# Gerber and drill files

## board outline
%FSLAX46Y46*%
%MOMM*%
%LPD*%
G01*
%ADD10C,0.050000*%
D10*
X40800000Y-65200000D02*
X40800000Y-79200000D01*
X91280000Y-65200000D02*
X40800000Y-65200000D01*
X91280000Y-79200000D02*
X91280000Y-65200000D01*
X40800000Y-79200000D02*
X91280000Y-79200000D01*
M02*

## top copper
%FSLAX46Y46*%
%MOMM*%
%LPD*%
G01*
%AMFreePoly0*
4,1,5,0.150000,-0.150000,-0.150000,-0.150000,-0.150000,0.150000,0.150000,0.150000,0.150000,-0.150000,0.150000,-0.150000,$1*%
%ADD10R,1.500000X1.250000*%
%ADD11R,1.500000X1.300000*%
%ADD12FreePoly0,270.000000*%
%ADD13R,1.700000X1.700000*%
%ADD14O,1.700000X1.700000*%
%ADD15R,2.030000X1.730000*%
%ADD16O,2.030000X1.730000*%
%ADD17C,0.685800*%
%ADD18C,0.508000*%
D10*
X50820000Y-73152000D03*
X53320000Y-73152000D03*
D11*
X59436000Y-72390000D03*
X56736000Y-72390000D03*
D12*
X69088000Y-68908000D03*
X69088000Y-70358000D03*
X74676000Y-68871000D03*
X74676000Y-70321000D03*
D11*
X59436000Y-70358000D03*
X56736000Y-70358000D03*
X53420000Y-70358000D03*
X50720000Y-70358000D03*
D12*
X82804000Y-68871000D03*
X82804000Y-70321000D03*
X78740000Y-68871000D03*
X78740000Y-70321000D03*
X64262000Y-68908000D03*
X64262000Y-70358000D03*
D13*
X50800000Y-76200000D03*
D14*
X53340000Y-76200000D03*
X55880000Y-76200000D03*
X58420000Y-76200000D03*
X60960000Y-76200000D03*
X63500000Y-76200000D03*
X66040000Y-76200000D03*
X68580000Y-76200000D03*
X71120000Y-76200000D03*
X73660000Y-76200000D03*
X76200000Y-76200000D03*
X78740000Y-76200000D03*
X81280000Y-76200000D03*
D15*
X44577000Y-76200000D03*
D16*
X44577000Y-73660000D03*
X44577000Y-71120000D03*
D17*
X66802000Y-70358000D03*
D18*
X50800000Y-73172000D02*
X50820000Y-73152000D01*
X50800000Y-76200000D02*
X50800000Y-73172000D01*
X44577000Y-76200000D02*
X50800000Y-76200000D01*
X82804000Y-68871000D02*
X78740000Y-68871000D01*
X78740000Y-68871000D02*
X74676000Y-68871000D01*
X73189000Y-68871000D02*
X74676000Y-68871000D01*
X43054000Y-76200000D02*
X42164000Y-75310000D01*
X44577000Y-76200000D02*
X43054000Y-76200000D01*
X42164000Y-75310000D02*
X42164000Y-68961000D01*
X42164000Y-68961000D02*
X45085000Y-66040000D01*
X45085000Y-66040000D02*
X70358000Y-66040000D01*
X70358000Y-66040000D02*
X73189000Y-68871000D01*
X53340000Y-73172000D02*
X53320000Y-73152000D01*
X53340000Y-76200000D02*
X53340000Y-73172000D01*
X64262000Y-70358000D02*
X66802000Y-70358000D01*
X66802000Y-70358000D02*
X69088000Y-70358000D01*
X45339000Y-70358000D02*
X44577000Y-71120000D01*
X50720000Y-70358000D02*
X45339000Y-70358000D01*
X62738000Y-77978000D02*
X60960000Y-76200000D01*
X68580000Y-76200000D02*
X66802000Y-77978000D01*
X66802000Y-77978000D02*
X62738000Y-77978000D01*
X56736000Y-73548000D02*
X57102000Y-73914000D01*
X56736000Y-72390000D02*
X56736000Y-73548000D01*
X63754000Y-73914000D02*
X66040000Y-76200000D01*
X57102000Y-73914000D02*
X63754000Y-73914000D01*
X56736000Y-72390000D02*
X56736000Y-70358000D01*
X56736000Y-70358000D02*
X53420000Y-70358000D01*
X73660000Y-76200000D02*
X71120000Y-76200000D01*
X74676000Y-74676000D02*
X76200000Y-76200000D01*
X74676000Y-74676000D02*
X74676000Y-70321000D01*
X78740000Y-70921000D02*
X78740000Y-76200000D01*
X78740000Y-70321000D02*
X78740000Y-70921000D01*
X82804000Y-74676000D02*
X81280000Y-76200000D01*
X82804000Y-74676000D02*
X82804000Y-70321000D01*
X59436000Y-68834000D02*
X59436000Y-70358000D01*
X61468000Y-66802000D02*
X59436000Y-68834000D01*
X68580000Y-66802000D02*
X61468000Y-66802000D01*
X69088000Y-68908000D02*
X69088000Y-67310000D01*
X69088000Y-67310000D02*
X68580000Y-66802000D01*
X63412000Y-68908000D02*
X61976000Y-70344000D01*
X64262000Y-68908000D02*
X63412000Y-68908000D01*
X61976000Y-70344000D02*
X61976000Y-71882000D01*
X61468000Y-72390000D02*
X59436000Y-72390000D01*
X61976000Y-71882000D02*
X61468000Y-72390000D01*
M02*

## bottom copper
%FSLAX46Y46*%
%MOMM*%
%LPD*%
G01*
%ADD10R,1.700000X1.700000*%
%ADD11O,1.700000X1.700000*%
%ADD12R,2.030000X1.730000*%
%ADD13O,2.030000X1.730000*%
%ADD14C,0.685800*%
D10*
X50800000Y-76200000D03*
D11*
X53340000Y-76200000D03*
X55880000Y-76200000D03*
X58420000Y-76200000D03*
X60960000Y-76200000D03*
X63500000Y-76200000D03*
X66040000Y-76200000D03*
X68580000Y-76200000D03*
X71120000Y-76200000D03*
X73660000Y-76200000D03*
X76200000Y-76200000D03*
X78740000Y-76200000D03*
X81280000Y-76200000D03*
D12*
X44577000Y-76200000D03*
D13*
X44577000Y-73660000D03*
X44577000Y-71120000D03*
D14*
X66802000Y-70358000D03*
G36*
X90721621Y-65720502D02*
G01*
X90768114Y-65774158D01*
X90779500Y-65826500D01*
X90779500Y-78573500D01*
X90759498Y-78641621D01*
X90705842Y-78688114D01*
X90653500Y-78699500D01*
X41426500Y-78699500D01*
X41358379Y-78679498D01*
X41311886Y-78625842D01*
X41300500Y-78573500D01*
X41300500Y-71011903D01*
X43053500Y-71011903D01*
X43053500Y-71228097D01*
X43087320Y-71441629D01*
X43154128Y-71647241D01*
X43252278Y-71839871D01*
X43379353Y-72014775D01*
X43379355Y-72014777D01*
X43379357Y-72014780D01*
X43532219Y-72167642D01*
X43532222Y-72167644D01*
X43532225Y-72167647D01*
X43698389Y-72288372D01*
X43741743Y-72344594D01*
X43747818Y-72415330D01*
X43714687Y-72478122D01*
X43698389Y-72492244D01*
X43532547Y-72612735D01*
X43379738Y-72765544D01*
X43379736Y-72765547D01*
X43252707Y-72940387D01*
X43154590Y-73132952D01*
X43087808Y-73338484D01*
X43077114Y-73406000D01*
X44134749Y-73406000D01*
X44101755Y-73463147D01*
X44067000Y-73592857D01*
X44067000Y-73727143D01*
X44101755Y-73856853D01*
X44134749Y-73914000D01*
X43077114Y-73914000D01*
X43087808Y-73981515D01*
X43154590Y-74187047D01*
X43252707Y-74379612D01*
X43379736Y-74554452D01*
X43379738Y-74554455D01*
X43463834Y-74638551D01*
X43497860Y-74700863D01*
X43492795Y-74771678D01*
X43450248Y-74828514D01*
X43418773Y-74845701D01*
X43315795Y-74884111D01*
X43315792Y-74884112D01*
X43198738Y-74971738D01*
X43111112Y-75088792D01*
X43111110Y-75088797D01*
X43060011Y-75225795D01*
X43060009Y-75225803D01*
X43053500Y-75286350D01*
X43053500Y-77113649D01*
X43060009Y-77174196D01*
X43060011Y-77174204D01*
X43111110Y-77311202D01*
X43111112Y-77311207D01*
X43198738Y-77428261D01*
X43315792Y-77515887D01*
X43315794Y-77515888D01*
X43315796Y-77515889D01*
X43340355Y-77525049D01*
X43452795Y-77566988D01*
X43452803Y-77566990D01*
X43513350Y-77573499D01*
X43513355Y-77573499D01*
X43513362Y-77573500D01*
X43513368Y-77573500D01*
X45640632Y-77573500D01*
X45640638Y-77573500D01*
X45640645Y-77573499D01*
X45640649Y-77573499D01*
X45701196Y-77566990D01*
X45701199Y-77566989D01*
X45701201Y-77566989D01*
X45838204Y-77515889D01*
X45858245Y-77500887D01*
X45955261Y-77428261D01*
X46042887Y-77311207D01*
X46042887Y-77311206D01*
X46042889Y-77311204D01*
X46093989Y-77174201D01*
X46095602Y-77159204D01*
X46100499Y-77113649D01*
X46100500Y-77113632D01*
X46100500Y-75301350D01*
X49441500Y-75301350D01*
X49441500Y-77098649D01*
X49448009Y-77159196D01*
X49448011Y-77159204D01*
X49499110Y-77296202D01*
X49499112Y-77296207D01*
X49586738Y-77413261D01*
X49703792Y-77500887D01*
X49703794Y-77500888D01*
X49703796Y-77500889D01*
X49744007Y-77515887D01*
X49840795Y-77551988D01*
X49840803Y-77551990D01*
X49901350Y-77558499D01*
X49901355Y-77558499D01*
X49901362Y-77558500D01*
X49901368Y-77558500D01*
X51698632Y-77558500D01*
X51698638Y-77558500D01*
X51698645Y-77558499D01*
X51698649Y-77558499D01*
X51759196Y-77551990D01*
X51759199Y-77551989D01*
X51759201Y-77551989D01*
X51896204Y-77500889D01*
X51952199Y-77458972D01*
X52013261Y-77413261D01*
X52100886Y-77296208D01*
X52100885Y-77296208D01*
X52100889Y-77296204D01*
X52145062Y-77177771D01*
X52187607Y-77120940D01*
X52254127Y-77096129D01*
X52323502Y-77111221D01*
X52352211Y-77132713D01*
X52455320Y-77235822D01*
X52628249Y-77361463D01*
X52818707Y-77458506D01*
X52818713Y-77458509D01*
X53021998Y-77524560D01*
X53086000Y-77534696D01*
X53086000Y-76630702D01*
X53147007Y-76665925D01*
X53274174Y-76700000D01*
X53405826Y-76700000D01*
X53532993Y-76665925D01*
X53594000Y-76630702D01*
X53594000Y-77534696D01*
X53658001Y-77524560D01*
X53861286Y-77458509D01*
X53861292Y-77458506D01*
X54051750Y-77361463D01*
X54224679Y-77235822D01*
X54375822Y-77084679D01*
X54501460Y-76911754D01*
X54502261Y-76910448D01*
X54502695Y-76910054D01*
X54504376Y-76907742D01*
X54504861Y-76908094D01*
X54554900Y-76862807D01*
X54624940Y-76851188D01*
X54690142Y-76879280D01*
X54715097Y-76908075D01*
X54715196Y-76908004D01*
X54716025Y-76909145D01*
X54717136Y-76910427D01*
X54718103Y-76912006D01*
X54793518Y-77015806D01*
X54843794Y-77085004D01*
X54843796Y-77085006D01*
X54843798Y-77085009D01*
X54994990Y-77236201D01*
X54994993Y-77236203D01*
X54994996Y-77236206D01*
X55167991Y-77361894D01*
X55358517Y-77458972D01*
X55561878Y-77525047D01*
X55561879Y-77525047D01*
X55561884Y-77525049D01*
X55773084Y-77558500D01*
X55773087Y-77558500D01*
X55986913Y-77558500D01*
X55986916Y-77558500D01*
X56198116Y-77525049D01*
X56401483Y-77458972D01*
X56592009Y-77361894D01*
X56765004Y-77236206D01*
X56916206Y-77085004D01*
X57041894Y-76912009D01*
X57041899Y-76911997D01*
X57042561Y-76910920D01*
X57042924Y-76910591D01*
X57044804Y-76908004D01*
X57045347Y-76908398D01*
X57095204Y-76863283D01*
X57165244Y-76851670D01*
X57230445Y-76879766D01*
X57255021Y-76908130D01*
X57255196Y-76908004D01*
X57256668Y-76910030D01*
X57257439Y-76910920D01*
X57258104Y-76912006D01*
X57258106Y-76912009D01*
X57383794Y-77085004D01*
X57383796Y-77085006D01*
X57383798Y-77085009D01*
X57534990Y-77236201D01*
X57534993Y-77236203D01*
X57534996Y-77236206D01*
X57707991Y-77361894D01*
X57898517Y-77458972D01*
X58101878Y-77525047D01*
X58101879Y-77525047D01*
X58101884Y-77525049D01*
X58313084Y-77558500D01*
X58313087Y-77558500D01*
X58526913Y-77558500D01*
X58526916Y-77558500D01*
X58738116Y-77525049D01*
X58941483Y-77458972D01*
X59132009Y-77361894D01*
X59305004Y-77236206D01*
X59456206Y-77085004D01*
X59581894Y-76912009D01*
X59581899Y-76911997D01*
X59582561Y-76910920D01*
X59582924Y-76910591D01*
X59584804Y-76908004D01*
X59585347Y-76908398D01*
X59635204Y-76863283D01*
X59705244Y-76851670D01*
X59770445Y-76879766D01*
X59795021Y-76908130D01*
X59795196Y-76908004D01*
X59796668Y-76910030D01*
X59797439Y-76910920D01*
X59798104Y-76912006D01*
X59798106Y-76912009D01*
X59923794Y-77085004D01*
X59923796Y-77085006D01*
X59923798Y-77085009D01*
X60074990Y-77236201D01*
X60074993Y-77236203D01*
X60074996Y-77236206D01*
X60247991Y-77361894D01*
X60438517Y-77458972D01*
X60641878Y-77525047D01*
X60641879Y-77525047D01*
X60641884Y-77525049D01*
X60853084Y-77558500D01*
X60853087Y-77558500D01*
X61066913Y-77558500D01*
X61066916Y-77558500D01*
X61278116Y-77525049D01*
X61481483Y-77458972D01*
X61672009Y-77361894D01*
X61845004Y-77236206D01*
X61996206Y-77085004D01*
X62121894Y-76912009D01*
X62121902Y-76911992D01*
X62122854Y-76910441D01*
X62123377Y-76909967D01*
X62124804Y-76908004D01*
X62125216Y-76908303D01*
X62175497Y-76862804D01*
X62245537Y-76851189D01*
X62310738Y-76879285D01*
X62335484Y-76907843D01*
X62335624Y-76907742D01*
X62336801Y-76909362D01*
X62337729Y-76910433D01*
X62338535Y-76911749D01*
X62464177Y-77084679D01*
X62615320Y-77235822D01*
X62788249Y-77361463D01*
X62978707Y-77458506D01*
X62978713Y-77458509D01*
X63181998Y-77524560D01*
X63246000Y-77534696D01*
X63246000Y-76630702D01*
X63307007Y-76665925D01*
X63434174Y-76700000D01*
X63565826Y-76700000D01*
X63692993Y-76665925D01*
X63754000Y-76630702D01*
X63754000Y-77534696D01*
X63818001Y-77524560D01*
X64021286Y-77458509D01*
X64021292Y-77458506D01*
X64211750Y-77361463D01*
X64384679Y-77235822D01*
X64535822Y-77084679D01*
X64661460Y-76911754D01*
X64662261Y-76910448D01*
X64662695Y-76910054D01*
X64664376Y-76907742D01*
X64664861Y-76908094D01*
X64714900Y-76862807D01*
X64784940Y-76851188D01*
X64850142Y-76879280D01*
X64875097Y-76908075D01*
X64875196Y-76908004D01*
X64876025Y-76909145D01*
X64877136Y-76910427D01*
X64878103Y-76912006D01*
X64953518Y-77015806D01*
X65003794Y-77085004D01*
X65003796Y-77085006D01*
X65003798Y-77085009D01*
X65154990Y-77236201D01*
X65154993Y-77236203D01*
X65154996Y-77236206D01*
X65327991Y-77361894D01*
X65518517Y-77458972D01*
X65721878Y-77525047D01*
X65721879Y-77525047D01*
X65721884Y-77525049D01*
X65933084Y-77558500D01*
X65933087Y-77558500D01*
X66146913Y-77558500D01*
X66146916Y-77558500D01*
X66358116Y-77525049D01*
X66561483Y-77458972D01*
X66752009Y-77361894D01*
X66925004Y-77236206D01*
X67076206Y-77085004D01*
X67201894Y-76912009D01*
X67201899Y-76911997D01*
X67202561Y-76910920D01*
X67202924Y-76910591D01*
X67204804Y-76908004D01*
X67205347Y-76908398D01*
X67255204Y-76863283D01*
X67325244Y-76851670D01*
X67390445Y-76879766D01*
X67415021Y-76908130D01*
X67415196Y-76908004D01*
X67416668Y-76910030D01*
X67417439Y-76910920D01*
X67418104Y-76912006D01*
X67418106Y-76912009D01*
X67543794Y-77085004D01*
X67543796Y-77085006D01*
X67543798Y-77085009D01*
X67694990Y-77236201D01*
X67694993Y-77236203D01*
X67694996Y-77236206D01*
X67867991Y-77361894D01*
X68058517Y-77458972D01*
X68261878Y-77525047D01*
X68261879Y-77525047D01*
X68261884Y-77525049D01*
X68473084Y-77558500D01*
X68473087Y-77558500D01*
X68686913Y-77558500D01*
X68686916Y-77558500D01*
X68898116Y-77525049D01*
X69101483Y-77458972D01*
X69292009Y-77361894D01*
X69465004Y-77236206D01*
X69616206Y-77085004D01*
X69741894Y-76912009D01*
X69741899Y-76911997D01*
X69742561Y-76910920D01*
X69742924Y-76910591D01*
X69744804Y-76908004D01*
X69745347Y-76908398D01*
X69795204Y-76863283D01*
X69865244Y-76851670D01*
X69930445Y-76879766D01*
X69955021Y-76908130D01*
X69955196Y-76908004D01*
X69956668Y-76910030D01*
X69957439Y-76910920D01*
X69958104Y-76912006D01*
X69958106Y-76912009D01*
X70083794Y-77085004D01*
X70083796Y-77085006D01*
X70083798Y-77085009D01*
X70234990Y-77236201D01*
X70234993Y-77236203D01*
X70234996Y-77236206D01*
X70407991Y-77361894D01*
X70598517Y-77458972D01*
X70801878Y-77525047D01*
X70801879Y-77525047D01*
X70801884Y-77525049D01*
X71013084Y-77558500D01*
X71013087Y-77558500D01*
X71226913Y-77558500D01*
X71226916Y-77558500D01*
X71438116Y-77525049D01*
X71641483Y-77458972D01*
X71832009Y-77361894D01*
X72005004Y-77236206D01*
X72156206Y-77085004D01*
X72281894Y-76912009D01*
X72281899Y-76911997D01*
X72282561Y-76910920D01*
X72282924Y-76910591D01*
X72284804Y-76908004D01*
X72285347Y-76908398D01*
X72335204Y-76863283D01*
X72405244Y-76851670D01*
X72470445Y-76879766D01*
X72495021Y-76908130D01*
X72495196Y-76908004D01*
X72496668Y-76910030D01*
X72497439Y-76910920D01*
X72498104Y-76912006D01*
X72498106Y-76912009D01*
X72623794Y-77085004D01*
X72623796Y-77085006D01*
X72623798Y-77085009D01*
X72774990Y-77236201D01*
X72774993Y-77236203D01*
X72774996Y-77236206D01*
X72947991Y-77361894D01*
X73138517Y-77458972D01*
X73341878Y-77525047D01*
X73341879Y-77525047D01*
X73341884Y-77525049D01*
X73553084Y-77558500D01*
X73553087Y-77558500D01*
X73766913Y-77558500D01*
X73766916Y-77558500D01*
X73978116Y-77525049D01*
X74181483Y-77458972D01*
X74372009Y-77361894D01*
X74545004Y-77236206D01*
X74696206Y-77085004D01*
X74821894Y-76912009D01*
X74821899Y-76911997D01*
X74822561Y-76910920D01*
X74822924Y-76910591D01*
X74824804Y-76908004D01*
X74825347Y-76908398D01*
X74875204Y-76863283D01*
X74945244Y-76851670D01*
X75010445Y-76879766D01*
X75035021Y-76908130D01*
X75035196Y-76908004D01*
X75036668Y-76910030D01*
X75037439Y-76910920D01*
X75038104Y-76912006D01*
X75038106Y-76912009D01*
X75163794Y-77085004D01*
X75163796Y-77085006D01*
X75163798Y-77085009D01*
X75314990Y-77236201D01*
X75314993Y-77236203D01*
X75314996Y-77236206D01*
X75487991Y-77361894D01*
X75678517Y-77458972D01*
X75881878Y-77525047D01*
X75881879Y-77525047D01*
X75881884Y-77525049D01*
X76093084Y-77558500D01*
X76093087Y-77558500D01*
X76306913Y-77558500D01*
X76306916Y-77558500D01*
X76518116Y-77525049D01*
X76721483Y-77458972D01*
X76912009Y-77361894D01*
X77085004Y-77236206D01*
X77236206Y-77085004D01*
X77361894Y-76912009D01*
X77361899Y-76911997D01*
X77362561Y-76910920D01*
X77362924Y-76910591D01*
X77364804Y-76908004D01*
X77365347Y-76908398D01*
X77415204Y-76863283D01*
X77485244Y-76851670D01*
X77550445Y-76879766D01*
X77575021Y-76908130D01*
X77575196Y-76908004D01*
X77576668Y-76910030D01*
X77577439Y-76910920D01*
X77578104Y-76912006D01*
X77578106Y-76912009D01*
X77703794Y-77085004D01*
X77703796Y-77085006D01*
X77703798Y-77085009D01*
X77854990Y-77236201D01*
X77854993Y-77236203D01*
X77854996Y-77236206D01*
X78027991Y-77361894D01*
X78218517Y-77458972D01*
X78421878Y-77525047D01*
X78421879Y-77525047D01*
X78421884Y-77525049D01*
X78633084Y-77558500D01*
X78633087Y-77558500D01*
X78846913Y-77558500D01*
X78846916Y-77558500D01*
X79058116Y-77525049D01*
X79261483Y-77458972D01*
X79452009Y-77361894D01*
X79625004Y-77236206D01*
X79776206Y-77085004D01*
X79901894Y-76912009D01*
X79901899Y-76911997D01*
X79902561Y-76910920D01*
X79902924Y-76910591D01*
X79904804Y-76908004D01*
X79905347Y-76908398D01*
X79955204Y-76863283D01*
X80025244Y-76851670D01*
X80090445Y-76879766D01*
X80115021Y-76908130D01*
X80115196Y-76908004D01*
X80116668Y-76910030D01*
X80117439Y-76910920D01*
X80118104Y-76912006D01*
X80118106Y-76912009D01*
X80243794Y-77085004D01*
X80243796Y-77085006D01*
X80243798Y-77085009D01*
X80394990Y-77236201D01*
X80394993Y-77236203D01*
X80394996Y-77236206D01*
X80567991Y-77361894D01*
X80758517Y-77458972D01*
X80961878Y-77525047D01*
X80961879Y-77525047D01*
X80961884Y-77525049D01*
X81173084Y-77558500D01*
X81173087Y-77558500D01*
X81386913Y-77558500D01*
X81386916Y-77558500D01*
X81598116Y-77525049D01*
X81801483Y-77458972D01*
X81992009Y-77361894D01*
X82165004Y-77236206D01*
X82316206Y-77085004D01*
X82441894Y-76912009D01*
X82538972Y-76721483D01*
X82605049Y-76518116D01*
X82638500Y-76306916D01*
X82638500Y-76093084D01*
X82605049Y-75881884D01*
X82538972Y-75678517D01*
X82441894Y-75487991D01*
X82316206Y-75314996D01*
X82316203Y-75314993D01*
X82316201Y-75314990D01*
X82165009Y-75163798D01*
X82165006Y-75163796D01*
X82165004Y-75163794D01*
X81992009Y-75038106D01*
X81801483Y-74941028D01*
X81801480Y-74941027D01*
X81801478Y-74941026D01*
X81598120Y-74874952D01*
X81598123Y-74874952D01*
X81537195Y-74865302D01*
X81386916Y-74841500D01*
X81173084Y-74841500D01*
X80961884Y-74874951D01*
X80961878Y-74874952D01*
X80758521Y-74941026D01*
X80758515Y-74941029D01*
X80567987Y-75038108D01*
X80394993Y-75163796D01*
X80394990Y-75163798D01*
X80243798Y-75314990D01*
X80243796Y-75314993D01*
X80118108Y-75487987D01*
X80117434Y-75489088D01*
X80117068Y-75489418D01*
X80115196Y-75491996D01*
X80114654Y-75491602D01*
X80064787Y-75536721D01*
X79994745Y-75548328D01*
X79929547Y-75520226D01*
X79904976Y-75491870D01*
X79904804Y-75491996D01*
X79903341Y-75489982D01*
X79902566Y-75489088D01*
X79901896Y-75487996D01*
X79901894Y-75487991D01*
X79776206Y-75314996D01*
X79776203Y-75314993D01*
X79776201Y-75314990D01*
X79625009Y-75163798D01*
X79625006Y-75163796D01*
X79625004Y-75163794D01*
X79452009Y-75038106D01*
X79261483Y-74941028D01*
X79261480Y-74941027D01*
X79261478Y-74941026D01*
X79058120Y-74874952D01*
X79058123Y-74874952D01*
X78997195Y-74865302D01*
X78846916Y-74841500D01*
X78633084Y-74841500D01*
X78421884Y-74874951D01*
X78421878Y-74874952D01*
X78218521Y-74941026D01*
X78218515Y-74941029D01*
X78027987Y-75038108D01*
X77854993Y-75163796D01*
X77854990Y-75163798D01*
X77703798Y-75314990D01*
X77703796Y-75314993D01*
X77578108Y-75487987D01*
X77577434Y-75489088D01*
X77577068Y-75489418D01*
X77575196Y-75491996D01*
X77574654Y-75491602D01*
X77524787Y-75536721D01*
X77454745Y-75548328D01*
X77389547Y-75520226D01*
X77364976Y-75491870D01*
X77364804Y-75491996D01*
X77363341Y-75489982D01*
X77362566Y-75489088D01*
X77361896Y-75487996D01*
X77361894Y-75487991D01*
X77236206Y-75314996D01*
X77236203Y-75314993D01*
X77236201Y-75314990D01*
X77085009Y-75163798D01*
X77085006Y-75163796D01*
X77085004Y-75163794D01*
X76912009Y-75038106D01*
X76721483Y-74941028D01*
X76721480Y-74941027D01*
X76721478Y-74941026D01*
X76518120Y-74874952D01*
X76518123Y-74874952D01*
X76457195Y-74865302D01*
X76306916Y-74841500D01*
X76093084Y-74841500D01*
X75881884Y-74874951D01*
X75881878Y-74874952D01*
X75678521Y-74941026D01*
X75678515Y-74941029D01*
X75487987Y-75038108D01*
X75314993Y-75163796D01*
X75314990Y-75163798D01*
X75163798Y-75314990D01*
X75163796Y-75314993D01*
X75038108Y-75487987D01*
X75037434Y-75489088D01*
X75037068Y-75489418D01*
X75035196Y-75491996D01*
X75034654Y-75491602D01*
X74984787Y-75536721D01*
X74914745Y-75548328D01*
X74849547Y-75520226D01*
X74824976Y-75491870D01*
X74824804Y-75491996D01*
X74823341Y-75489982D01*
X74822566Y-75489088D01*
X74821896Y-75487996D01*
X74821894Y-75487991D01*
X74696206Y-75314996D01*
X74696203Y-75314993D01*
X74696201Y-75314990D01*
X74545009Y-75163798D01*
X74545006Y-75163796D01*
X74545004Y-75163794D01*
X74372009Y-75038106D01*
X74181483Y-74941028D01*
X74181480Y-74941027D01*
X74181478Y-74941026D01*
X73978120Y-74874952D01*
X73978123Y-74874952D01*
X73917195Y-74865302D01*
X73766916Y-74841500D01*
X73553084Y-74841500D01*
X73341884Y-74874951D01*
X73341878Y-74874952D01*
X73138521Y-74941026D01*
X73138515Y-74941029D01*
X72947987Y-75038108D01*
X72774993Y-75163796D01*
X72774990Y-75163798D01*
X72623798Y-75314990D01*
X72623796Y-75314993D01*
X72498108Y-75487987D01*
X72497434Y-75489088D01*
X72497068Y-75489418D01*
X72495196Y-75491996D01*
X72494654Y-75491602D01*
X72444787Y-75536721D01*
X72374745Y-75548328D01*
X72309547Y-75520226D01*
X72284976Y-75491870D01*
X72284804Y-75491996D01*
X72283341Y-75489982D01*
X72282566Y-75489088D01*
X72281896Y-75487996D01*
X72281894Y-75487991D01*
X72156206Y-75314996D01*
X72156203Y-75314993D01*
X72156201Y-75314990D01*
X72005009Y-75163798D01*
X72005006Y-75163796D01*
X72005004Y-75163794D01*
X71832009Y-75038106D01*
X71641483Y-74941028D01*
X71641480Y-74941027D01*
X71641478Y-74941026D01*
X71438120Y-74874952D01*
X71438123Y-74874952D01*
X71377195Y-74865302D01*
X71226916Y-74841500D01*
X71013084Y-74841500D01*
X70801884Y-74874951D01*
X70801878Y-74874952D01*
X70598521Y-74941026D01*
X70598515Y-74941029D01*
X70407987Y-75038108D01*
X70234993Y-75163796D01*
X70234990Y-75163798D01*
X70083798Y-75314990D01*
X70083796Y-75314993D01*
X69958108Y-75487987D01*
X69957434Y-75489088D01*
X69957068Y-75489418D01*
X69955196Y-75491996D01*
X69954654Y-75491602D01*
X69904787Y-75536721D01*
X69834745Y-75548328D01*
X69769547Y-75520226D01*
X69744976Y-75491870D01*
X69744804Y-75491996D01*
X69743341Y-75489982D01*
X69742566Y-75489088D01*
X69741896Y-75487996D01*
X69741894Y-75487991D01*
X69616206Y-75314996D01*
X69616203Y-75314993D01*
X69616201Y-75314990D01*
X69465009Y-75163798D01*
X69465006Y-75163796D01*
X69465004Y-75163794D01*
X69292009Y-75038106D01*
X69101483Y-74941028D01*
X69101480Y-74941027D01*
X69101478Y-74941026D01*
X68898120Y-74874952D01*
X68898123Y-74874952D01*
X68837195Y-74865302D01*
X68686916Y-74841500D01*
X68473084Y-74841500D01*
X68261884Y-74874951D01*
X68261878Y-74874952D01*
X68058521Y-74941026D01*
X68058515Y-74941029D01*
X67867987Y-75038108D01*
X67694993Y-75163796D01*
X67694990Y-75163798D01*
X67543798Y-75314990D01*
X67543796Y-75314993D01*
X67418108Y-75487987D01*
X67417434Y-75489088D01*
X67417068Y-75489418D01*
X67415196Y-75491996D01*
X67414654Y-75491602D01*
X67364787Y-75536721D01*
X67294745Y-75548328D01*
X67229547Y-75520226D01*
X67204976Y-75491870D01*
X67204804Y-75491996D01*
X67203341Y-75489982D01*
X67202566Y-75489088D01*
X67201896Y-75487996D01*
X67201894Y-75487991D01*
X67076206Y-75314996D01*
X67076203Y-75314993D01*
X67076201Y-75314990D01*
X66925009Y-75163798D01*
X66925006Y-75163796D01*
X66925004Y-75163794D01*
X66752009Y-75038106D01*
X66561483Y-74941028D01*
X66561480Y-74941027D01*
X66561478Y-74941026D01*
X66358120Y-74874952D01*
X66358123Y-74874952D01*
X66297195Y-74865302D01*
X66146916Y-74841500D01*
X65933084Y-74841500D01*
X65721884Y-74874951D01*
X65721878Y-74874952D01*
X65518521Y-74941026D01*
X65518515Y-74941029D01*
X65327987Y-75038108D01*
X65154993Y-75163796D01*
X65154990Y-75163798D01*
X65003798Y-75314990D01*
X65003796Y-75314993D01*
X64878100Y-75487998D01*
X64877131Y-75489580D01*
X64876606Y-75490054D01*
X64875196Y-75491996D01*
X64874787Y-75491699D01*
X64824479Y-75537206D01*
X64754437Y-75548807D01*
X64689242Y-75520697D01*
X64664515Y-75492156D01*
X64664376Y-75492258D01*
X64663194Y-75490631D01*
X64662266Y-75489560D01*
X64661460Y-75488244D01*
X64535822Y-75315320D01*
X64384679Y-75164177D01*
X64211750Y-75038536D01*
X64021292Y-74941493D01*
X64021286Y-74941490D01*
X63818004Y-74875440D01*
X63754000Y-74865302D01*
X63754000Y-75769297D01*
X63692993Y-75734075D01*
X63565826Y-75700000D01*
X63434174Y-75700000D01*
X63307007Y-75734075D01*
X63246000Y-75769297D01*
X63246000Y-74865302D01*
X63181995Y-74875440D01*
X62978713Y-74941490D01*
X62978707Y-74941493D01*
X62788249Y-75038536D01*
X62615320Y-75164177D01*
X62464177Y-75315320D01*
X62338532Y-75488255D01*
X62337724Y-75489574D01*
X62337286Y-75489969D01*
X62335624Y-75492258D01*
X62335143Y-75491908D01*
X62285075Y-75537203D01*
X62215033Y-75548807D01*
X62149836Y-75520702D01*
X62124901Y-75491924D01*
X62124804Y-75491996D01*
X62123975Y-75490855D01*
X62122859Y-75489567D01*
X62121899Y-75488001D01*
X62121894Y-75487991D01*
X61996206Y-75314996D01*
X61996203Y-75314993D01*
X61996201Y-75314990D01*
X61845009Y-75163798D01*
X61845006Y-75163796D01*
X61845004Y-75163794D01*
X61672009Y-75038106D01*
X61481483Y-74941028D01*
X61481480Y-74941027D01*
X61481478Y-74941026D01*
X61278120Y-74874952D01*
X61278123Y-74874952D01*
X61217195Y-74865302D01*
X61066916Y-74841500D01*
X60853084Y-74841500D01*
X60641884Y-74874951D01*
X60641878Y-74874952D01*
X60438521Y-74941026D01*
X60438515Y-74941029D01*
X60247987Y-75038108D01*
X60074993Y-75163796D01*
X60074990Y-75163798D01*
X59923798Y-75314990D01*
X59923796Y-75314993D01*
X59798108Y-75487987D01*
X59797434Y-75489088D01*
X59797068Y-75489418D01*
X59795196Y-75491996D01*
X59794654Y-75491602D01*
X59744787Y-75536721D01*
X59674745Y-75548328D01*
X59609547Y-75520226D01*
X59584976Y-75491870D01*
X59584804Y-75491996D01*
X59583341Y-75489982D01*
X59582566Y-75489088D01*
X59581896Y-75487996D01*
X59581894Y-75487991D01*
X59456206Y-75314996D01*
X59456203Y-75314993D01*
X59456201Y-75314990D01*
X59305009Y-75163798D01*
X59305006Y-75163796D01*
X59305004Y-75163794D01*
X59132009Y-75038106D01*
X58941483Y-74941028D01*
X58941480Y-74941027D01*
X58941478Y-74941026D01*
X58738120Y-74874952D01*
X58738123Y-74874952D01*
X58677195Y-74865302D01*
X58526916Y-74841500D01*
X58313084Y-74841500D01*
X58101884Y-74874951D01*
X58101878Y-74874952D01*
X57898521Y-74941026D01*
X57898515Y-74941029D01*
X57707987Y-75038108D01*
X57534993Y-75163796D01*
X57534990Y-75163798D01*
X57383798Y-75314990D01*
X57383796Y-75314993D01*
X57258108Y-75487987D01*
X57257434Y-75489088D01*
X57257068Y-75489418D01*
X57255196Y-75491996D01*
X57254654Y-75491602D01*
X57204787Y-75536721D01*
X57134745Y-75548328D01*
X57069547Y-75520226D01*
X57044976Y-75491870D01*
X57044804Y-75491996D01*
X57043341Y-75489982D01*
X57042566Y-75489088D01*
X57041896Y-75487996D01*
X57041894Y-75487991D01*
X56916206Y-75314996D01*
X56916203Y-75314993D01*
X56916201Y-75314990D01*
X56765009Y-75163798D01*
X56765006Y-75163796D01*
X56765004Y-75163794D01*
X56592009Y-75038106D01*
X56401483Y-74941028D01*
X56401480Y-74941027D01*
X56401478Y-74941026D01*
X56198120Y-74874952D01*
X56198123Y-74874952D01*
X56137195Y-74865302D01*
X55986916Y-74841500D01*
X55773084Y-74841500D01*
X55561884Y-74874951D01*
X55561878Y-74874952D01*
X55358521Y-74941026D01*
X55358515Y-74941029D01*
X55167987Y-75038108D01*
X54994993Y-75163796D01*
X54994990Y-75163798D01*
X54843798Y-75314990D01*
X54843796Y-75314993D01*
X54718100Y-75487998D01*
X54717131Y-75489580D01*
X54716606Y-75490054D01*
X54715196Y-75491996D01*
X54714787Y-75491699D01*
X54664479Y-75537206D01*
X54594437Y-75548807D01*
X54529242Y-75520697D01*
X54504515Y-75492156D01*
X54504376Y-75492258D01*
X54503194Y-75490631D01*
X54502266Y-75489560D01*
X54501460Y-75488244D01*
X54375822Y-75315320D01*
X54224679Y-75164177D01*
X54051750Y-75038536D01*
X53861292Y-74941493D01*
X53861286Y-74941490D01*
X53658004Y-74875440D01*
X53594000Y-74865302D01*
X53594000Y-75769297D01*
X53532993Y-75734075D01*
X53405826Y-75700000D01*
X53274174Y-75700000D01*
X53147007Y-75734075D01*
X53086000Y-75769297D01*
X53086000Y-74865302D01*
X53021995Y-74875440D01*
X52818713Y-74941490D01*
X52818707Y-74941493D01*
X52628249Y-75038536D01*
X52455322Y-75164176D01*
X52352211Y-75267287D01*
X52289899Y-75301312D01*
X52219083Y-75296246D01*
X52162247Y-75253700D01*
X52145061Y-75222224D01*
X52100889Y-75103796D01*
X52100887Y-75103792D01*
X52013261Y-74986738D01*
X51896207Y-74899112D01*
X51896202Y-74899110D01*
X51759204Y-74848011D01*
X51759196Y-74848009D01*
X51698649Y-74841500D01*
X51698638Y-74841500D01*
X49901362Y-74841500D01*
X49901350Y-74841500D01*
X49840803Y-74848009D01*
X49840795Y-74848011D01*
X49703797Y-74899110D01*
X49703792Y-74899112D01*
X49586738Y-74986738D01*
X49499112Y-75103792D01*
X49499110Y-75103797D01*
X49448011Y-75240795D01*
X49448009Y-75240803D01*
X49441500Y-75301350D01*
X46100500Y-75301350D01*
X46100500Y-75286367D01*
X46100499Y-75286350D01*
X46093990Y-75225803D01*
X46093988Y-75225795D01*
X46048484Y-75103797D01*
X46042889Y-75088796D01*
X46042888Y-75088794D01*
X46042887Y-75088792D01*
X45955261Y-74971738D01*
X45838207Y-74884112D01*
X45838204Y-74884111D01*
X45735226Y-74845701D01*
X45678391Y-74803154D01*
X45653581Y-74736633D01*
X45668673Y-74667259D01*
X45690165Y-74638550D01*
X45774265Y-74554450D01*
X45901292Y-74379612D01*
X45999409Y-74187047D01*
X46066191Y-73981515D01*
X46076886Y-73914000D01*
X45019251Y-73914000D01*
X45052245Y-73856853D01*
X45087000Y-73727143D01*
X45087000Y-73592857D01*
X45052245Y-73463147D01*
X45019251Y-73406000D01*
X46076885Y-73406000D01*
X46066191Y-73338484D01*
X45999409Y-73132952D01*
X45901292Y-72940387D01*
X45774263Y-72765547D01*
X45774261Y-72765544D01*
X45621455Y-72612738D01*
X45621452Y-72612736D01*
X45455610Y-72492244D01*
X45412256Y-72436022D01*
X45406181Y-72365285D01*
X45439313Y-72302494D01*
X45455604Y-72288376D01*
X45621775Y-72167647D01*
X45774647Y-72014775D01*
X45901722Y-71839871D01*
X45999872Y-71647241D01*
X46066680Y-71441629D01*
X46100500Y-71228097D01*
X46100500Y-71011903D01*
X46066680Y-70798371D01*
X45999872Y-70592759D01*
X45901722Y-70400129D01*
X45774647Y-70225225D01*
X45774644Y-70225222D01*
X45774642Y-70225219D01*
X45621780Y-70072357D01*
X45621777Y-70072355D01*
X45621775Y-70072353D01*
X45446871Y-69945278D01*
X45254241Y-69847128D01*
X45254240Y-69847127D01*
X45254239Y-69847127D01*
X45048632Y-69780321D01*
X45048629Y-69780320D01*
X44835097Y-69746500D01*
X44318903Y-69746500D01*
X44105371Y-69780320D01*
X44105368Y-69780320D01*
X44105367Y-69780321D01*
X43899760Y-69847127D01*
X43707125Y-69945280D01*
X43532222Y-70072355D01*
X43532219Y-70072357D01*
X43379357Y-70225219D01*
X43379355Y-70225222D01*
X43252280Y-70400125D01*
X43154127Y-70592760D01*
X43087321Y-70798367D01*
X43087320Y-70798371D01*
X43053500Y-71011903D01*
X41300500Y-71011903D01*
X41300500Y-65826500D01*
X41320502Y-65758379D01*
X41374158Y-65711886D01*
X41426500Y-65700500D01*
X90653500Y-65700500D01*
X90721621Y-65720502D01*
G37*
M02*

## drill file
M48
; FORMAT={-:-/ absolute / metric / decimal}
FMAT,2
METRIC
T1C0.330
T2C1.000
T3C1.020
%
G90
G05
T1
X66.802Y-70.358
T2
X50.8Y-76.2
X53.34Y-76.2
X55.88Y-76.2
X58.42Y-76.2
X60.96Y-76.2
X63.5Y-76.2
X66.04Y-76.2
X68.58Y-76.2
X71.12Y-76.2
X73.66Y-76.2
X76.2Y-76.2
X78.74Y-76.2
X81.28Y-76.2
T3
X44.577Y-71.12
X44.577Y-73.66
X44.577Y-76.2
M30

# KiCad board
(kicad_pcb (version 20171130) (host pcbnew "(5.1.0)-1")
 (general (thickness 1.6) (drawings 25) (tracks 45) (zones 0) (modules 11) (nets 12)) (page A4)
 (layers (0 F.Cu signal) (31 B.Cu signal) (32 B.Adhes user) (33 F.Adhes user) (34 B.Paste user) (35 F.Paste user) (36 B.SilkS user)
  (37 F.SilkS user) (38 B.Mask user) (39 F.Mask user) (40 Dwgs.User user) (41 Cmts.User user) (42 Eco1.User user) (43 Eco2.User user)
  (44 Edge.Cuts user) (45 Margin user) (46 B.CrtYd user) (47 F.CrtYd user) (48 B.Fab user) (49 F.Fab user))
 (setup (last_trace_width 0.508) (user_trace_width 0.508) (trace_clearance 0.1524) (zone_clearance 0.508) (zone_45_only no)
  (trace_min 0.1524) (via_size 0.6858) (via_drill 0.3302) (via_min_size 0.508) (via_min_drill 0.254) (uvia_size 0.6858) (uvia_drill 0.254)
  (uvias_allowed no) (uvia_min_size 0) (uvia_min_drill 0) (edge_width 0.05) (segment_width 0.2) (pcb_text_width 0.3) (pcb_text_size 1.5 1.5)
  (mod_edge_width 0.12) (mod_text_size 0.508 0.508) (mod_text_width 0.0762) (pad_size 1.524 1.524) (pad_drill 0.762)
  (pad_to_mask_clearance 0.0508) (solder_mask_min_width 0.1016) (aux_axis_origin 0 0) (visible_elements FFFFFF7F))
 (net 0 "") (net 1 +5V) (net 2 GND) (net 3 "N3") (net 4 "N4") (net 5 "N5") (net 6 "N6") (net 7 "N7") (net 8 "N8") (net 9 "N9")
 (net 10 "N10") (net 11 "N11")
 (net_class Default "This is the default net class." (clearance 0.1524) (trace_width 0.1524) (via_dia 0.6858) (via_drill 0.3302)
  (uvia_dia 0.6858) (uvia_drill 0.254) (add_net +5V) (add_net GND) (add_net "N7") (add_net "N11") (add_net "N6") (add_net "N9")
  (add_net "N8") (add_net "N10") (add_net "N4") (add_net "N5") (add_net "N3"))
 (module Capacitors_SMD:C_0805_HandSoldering (layer F.Cu) (at 52.07 73.152)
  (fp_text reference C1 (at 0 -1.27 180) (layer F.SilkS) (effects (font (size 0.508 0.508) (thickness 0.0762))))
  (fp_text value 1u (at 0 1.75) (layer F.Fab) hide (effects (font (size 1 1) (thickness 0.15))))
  (pad 1 smd rect (at -1.25 0) (size 1.5 1.25) (layers F.Cu F.Paste F.Mask) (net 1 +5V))
  (pad 2 smd rect (at 1.25 0) (size 1.5 1.25) (layers F.Cu F.Paste F.Mask) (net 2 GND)))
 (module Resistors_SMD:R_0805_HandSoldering (layer F.Cu) (at 58.086 72.39 180)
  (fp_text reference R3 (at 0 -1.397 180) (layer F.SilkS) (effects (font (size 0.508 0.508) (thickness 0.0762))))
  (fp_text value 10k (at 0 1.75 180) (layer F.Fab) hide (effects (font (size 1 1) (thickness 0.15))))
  (pad 1 smd rect (at -1.35 0 180) (size 1.5 1.3) (layers F.Cu F.Paste F.Mask) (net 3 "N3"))
  (pad 2 smd rect (at 1.35 0 180) (size 1.5 1.3) (layers F.Cu F.Paste F.Mask) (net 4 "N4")))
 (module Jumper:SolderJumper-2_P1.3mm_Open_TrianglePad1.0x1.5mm (layer F.Cu) (at 69.088 69.633 270)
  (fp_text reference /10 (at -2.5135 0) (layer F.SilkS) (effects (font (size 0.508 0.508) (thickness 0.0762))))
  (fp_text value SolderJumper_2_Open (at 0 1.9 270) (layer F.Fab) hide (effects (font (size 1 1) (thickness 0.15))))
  (pad 1 smd custom (at -0.725 0 270) (size 0.3 0.3) (layers F.Cu F.Mask) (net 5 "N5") (zone_connect 2)
   (options (clearance outline) (anchor rect)) (primitives))
  (pad 2 smd custom (at 0.725 0 270) (size 0.3 0.3) (layers F.Cu F.Mask) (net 2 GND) (zone_connect 2)
   (options (clearance outline) (anchor rect)) (primitives)))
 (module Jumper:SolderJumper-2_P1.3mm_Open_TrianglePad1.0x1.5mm (layer F.Cu) (at 74.676 69.596 270)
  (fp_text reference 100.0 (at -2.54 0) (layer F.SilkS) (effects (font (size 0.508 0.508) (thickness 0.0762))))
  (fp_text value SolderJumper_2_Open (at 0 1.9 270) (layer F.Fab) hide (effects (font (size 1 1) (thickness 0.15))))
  (pad 1 smd custom (at -0.725 0 270) (size 0.3 0.3) (layers F.Cu F.Mask) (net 1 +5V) (zone_connect 2)
   (options (clearance outline) (anchor rect)) (primitives))
  (pad 2 smd custom (at 0.725 0 270) (size 0.3 0.3) (layers F.Cu F.Mask) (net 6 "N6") (zone_connect 2)
   (options (clearance outline) (anchor rect)) (primitives)))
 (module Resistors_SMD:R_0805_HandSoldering (layer F.Cu) (at 58.086 70.358 180)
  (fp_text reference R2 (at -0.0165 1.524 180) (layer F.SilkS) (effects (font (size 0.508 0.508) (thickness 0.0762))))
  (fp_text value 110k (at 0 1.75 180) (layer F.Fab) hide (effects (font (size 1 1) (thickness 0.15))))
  (pad 1 smd rect (at -1.35 0 180) (size 1.5 1.3) (layers F.Cu F.Paste F.Mask) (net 5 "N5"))
  (pad 2 smd rect (at 1.35 0 180) (size 1.5 1.3) (layers F.Cu F.Paste F.Mask) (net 4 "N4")))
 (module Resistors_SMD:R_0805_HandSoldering (layer F.Cu) (at 52.07 70.358 180)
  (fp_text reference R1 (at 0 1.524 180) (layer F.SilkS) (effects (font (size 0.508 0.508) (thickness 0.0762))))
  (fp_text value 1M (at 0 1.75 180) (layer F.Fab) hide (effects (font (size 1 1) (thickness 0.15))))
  (pad 1 smd rect (at -1.35 0 180) (size 1.5 1.3) (layers F.Cu F.Paste F.Mask) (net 4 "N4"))
  (pad 2 smd rect (at 1.35 0 180) (size 1.5 1.3) (layers F.Cu F.Paste F.Mask) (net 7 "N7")))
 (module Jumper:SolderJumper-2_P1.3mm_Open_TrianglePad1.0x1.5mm (layer F.Cu) (at 82.804 69.596 270)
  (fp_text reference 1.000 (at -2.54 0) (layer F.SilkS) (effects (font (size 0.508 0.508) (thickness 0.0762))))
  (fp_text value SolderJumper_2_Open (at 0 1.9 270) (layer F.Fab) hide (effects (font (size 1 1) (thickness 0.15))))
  (pad 1 smd custom (at -0.725 0 270) (size 0.3 0.3) (layers F.Cu F.Mask) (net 1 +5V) (zone_connect 2)
   (options (clearance outline) (anchor rect)) (primitives))
  (pad 2 smd custom (at 0.725 0 270) (size 0.3 0.3) (layers F.Cu F.Mask) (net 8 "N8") (zone_connect 2)
   (options (clearance outline) (anchor rect)) (primitives)))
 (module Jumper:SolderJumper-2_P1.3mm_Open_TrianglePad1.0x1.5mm (layer F.Cu) (at 78.74 69.596 270)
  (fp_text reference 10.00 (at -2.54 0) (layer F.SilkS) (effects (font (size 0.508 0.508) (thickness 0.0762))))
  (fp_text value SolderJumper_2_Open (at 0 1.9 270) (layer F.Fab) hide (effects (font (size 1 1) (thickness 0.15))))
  (pad 1 smd custom (at -0.725 0 270) (size 0.3 0.3) (layers F.Cu F.Mask) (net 1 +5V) (zone_connect 2)
   (options (clearance outline) (anchor rect)) (primitives))
  (pad 2 smd custom (at 0.725 0 270) (size 0.3 0.3) (layers F.Cu F.Mask) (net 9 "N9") (zone_connect 2)
   (options (clearance outline) (anchor rect)) (primitives)))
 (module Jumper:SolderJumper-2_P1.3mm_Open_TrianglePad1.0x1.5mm (layer F.Cu) (at 64.262 69.633 270)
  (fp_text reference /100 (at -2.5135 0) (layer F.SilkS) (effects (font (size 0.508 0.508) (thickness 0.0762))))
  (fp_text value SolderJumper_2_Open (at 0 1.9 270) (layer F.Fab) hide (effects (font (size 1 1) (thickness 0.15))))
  (pad 1 smd custom (at -0.725 0 270) (size 0.3 0.3) (layers F.Cu F.Mask) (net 3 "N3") (zone_connect 2)
   (options (clearance outline) (anchor rect)) (primitives))
  (pad 2 smd custom (at 0.725 0 270) (size 0.3 0.3) (layers F.Cu F.Mask) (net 2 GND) (zone_connect 2)
   (options (clearance outline) (anchor rect)) (primitives)))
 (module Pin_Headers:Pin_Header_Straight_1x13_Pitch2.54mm (layer F.Cu) (at 50.8 76.2 90)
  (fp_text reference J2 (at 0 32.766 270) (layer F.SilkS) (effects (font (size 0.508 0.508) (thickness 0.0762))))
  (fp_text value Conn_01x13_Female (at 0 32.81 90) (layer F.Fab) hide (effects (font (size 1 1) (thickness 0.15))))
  (pad 1 thru_hole rect (at 0 0 90) (size 1.7 1.7) (drill 1) (layers *.Cu *.Mask) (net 1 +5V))
  (pad 2 thru_hole oval (at 0 2.54 90) (size 1.7 1.7) (drill 1) (layers *.Cu *.Mask) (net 2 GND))
  (pad 3 thru_hole oval (at 0 5.08 90) (size 1.7 1.7) (drill 1) (layers *.Cu *.Mask))
  (pad 4 thru_hole oval (at 0 7.62 90) (size 1.7 1.7) (drill 1) (layers *.Cu *.Mask))
  (pad 5 thru_hole oval (at 0 10.16 90) (size 1.7 1.7) (drill 1) (layers *.Cu *.Mask) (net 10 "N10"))
  (pad 6 thru_hole oval (at 0 12.7 90) (size 1.7 1.7) (drill 1) (layers *.Cu *.Mask) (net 2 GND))
  (pad 7 thru_hole oval (at 0 15.24 90) (size 1.7 1.7) (drill 1) (layers *.Cu *.Mask) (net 4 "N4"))
  (pad 8 thru_hole oval (at 0 17.78 90) (size 1.7 1.7) (drill 1) (layers *.Cu *.Mask) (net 10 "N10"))
  (pad 9 thru_hole oval (at 0 20.32 90) (size 1.7 1.7) (drill 1) (layers *.Cu *.Mask) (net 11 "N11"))
  (pad 10 thru_hole oval (at 0 22.86 90) (size 1.7 1.7) (drill 1) (layers *.Cu *.Mask) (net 11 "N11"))
  (pad 11 thru_hole oval (at 0 25.4 90) (size 1.7 1.7) (drill 1) (layers *.Cu *.Mask) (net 6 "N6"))
  (pad 12 thru_hole oval (at 0 27.94 90) (size 1.7 1.7) (drill 1) (layers *.Cu *.Mask) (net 9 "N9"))
  (pad 13 thru_hole oval (at 0 30.48 90) (size 1.7 1.7) (drill 1) (layers *.Cu *.Mask) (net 8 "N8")))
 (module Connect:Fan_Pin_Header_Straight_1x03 (layer F.Cu) (at 44.577 76.2 180)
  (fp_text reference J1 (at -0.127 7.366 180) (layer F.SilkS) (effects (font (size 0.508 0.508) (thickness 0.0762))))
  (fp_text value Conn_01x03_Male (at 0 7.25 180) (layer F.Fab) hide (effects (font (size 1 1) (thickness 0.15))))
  (pad 1 thru_hole rect (at 0 0 180) (size 2.03 1.73) (drill 1.02) (layers *.Cu *.Mask) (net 1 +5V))
  (pad 2 thru_hole oval (at 0 2.54 180) (size 2.03 1.73) (drill 1.02) (layers *.Cu *.Mask) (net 2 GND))
  (pad 3 thru_hole oval (at 0 5.08 180) (size 2.03 1.73) (drill 1.02) (layers *.Cu *.Mask) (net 7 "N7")))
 (gr_line (start 40.8 65.2) (end 40.8 79.2) (layer Edge.Cuts) (width 0.05))
 (gr_line (start 91.28 65.2) (end 40.8 65.2) (layer Edge.Cuts) (width 0.05))
 (gr_line (start 91.28 79.2) (end 91.28 65.2) (layer Edge.Cuts) (width 0.05))
 (gr_line (start 40.8 79.2) (end 91.28 79.2) (layer Edge.Cuts) (width 0.05))
 (segment (start 50.8 73.172) (end 50.82 73.152) (width 0.508) (layer F.Cu) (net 1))
 (segment (start 50.8 76.2) (end 50.8 73.172) (width 0.508) (layer F.Cu) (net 1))
 (segment (start 44.577 76.2) (end 50.8 76.2) (width 0.508) (layer F.Cu) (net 1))
 (segment (start 82.804 68.871) (end 78.74 68.871) (width 0.508) (layer F.Cu) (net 1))
 (segment (start 78.74 68.871) (end 74.676 68.871) (width 0.508) (layer F.Cu) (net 1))
 (segment (start 73.189 68.871) (end 74.676 68.871) (width 0.508) (layer F.Cu) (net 1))
 (segment (start 43.054 76.2) (end 42.164 75.31) (width 0.508) (layer F.Cu) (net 1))
 (segment (start 44.577 76.2) (end 43.054 76.2) (width 0.508) (layer F.Cu) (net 1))
 (segment (start 42.164 75.31) (end 42.164 68.961) (width 0.508) (layer F.Cu) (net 1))
 (segment (start 42.164 68.961) (end 45.085 66.04) (width 0.508) (layer F.Cu) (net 1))
 (segment (start 45.085 66.04) (end 70.358 66.04) (width 0.508) (layer F.Cu) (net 1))
 (segment (start 70.358 66.04) (end 73.189 68.871) (width 0.508) (layer F.Cu) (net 1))
 (segment (start 53.34 73.172) (end 53.32 73.152) (width 0.508) (layer F.Cu) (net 2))
 (segment (start 53.34 76.2) (end 53.34 73.172) (width 0.508) (layer F.Cu) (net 2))
 (via (at 66.802 70.358) (size 0.6858) (drill 0.3302) (layers F.Cu B.Cu) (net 2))
 (segment (start 64.262 70.358) (end 66.802 70.358) (width 0.508) (layer F.Cu) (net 2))
 (segment (start 66.802 70.358) (end 69.088 70.358) (width 0.508) (layer F.Cu) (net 2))
 (segment (start 45.339 70.358) (end 44.577 71.12) (width 0.508) (layer F.Cu) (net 7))
 (segment (start 50.72 70.358) (end 45.339 70.358) (width 0.508) (layer F.Cu) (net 7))
 (segment (start 62.738 77.978) (end 60.96 76.2) (width 0.508) (layer F.Cu) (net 10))
 (segment (start 68.58 76.2) (end 66.802 77.978) (width 0.508) (layer F.Cu) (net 10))
 (segment (start 66.802 77.978) (end 62.738 77.978) (width 0.508) (layer F.Cu) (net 10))
 (segment (start 56.736 73.548) (end 57.102 73.914) (width 0.508) (layer F.Cu) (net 4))
 (segment (start 56.736 72.39) (end 56.736 73.548) (width 0.508) (layer F.Cu) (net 4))
 (segment (start 63.754 73.914) (end 66.04 76.2) (width 0.508) (layer F.Cu) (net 4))
 (segment (start 57.102 73.914) (end 63.754 73.914) (width 0.508) (layer F.Cu) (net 4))
 (segment (start 56.736 72.39) (end 56.736 70.358) (width 0.508) (layer F.Cu) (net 4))
 (segment (start 56.736 70.358) (end 53.42 70.358) (width 0.508) (layer F.Cu) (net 4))
 (segment (start 73.66 76.2) (end 71.12 76.2) (width 0.508) (layer F.Cu) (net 11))
 (segment (start 74.676 74.676) (end 76.2 76.2) (width 0.508) (layer F.Cu) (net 6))
 (segment (start 74.676 74.676) (end 74.676 70.321) (width 0.508) (layer F.Cu) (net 6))
 (segment (start 78.74 70.921) (end 78.74 76.2) (width 0.508) (layer F.Cu) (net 9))
 (segment (start 78.74 70.321) (end 78.74 70.921) (width 0.508) (layer F.Cu) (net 9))
 (segment (start 82.804 74.676) (end 81.28 76.2) (width 0.508) (layer F.Cu) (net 8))
 (segment (start 82.804 74.676) (end 82.804 70.321) (width 0.508) (layer F.Cu) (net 8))
 (segment (start 59.436 68.834) (end 59.436 70.358) (width 0.508) (layer F.Cu) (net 5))
 (segment (start 61.468 66.802) (end 59.436 68.834) (width 0.508) (layer F.Cu) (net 5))
 (segment (start 68.58 66.802) (end 61.468 66.802) (width 0.508) (layer F.Cu) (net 5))
 (segment (start 69.088 68.908) (end 69.088 67.31) (width 0.508) (layer F.Cu) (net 5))
 (segment (start 69.088 67.31) (end 68.58 66.802) (width 0.508) (layer F.Cu) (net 5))
 (segment (start 63.412 68.908) (end 61.976 70.344) (width 0.508) (layer F.Cu) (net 3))
 (segment (start 64.262 68.908) (end 63.412 68.908) (width 0.508) (layer F.Cu) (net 3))
 (segment (start 61.976 70.344) (end 61.976 71.882) (width 0.508) (layer F.Cu) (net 3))
 (segment (start 61.468 72.39) (end 59.436 72.39) (width 0.508) (layer F.Cu) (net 3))
 (segment (start 61.976 71.882) (end 61.468 72.39) (width 0.508) (layer F.Cu) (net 3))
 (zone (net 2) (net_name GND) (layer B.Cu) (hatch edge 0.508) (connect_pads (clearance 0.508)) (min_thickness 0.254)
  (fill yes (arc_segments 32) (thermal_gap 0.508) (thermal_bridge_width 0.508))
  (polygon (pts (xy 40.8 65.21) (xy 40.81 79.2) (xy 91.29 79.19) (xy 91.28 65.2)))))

